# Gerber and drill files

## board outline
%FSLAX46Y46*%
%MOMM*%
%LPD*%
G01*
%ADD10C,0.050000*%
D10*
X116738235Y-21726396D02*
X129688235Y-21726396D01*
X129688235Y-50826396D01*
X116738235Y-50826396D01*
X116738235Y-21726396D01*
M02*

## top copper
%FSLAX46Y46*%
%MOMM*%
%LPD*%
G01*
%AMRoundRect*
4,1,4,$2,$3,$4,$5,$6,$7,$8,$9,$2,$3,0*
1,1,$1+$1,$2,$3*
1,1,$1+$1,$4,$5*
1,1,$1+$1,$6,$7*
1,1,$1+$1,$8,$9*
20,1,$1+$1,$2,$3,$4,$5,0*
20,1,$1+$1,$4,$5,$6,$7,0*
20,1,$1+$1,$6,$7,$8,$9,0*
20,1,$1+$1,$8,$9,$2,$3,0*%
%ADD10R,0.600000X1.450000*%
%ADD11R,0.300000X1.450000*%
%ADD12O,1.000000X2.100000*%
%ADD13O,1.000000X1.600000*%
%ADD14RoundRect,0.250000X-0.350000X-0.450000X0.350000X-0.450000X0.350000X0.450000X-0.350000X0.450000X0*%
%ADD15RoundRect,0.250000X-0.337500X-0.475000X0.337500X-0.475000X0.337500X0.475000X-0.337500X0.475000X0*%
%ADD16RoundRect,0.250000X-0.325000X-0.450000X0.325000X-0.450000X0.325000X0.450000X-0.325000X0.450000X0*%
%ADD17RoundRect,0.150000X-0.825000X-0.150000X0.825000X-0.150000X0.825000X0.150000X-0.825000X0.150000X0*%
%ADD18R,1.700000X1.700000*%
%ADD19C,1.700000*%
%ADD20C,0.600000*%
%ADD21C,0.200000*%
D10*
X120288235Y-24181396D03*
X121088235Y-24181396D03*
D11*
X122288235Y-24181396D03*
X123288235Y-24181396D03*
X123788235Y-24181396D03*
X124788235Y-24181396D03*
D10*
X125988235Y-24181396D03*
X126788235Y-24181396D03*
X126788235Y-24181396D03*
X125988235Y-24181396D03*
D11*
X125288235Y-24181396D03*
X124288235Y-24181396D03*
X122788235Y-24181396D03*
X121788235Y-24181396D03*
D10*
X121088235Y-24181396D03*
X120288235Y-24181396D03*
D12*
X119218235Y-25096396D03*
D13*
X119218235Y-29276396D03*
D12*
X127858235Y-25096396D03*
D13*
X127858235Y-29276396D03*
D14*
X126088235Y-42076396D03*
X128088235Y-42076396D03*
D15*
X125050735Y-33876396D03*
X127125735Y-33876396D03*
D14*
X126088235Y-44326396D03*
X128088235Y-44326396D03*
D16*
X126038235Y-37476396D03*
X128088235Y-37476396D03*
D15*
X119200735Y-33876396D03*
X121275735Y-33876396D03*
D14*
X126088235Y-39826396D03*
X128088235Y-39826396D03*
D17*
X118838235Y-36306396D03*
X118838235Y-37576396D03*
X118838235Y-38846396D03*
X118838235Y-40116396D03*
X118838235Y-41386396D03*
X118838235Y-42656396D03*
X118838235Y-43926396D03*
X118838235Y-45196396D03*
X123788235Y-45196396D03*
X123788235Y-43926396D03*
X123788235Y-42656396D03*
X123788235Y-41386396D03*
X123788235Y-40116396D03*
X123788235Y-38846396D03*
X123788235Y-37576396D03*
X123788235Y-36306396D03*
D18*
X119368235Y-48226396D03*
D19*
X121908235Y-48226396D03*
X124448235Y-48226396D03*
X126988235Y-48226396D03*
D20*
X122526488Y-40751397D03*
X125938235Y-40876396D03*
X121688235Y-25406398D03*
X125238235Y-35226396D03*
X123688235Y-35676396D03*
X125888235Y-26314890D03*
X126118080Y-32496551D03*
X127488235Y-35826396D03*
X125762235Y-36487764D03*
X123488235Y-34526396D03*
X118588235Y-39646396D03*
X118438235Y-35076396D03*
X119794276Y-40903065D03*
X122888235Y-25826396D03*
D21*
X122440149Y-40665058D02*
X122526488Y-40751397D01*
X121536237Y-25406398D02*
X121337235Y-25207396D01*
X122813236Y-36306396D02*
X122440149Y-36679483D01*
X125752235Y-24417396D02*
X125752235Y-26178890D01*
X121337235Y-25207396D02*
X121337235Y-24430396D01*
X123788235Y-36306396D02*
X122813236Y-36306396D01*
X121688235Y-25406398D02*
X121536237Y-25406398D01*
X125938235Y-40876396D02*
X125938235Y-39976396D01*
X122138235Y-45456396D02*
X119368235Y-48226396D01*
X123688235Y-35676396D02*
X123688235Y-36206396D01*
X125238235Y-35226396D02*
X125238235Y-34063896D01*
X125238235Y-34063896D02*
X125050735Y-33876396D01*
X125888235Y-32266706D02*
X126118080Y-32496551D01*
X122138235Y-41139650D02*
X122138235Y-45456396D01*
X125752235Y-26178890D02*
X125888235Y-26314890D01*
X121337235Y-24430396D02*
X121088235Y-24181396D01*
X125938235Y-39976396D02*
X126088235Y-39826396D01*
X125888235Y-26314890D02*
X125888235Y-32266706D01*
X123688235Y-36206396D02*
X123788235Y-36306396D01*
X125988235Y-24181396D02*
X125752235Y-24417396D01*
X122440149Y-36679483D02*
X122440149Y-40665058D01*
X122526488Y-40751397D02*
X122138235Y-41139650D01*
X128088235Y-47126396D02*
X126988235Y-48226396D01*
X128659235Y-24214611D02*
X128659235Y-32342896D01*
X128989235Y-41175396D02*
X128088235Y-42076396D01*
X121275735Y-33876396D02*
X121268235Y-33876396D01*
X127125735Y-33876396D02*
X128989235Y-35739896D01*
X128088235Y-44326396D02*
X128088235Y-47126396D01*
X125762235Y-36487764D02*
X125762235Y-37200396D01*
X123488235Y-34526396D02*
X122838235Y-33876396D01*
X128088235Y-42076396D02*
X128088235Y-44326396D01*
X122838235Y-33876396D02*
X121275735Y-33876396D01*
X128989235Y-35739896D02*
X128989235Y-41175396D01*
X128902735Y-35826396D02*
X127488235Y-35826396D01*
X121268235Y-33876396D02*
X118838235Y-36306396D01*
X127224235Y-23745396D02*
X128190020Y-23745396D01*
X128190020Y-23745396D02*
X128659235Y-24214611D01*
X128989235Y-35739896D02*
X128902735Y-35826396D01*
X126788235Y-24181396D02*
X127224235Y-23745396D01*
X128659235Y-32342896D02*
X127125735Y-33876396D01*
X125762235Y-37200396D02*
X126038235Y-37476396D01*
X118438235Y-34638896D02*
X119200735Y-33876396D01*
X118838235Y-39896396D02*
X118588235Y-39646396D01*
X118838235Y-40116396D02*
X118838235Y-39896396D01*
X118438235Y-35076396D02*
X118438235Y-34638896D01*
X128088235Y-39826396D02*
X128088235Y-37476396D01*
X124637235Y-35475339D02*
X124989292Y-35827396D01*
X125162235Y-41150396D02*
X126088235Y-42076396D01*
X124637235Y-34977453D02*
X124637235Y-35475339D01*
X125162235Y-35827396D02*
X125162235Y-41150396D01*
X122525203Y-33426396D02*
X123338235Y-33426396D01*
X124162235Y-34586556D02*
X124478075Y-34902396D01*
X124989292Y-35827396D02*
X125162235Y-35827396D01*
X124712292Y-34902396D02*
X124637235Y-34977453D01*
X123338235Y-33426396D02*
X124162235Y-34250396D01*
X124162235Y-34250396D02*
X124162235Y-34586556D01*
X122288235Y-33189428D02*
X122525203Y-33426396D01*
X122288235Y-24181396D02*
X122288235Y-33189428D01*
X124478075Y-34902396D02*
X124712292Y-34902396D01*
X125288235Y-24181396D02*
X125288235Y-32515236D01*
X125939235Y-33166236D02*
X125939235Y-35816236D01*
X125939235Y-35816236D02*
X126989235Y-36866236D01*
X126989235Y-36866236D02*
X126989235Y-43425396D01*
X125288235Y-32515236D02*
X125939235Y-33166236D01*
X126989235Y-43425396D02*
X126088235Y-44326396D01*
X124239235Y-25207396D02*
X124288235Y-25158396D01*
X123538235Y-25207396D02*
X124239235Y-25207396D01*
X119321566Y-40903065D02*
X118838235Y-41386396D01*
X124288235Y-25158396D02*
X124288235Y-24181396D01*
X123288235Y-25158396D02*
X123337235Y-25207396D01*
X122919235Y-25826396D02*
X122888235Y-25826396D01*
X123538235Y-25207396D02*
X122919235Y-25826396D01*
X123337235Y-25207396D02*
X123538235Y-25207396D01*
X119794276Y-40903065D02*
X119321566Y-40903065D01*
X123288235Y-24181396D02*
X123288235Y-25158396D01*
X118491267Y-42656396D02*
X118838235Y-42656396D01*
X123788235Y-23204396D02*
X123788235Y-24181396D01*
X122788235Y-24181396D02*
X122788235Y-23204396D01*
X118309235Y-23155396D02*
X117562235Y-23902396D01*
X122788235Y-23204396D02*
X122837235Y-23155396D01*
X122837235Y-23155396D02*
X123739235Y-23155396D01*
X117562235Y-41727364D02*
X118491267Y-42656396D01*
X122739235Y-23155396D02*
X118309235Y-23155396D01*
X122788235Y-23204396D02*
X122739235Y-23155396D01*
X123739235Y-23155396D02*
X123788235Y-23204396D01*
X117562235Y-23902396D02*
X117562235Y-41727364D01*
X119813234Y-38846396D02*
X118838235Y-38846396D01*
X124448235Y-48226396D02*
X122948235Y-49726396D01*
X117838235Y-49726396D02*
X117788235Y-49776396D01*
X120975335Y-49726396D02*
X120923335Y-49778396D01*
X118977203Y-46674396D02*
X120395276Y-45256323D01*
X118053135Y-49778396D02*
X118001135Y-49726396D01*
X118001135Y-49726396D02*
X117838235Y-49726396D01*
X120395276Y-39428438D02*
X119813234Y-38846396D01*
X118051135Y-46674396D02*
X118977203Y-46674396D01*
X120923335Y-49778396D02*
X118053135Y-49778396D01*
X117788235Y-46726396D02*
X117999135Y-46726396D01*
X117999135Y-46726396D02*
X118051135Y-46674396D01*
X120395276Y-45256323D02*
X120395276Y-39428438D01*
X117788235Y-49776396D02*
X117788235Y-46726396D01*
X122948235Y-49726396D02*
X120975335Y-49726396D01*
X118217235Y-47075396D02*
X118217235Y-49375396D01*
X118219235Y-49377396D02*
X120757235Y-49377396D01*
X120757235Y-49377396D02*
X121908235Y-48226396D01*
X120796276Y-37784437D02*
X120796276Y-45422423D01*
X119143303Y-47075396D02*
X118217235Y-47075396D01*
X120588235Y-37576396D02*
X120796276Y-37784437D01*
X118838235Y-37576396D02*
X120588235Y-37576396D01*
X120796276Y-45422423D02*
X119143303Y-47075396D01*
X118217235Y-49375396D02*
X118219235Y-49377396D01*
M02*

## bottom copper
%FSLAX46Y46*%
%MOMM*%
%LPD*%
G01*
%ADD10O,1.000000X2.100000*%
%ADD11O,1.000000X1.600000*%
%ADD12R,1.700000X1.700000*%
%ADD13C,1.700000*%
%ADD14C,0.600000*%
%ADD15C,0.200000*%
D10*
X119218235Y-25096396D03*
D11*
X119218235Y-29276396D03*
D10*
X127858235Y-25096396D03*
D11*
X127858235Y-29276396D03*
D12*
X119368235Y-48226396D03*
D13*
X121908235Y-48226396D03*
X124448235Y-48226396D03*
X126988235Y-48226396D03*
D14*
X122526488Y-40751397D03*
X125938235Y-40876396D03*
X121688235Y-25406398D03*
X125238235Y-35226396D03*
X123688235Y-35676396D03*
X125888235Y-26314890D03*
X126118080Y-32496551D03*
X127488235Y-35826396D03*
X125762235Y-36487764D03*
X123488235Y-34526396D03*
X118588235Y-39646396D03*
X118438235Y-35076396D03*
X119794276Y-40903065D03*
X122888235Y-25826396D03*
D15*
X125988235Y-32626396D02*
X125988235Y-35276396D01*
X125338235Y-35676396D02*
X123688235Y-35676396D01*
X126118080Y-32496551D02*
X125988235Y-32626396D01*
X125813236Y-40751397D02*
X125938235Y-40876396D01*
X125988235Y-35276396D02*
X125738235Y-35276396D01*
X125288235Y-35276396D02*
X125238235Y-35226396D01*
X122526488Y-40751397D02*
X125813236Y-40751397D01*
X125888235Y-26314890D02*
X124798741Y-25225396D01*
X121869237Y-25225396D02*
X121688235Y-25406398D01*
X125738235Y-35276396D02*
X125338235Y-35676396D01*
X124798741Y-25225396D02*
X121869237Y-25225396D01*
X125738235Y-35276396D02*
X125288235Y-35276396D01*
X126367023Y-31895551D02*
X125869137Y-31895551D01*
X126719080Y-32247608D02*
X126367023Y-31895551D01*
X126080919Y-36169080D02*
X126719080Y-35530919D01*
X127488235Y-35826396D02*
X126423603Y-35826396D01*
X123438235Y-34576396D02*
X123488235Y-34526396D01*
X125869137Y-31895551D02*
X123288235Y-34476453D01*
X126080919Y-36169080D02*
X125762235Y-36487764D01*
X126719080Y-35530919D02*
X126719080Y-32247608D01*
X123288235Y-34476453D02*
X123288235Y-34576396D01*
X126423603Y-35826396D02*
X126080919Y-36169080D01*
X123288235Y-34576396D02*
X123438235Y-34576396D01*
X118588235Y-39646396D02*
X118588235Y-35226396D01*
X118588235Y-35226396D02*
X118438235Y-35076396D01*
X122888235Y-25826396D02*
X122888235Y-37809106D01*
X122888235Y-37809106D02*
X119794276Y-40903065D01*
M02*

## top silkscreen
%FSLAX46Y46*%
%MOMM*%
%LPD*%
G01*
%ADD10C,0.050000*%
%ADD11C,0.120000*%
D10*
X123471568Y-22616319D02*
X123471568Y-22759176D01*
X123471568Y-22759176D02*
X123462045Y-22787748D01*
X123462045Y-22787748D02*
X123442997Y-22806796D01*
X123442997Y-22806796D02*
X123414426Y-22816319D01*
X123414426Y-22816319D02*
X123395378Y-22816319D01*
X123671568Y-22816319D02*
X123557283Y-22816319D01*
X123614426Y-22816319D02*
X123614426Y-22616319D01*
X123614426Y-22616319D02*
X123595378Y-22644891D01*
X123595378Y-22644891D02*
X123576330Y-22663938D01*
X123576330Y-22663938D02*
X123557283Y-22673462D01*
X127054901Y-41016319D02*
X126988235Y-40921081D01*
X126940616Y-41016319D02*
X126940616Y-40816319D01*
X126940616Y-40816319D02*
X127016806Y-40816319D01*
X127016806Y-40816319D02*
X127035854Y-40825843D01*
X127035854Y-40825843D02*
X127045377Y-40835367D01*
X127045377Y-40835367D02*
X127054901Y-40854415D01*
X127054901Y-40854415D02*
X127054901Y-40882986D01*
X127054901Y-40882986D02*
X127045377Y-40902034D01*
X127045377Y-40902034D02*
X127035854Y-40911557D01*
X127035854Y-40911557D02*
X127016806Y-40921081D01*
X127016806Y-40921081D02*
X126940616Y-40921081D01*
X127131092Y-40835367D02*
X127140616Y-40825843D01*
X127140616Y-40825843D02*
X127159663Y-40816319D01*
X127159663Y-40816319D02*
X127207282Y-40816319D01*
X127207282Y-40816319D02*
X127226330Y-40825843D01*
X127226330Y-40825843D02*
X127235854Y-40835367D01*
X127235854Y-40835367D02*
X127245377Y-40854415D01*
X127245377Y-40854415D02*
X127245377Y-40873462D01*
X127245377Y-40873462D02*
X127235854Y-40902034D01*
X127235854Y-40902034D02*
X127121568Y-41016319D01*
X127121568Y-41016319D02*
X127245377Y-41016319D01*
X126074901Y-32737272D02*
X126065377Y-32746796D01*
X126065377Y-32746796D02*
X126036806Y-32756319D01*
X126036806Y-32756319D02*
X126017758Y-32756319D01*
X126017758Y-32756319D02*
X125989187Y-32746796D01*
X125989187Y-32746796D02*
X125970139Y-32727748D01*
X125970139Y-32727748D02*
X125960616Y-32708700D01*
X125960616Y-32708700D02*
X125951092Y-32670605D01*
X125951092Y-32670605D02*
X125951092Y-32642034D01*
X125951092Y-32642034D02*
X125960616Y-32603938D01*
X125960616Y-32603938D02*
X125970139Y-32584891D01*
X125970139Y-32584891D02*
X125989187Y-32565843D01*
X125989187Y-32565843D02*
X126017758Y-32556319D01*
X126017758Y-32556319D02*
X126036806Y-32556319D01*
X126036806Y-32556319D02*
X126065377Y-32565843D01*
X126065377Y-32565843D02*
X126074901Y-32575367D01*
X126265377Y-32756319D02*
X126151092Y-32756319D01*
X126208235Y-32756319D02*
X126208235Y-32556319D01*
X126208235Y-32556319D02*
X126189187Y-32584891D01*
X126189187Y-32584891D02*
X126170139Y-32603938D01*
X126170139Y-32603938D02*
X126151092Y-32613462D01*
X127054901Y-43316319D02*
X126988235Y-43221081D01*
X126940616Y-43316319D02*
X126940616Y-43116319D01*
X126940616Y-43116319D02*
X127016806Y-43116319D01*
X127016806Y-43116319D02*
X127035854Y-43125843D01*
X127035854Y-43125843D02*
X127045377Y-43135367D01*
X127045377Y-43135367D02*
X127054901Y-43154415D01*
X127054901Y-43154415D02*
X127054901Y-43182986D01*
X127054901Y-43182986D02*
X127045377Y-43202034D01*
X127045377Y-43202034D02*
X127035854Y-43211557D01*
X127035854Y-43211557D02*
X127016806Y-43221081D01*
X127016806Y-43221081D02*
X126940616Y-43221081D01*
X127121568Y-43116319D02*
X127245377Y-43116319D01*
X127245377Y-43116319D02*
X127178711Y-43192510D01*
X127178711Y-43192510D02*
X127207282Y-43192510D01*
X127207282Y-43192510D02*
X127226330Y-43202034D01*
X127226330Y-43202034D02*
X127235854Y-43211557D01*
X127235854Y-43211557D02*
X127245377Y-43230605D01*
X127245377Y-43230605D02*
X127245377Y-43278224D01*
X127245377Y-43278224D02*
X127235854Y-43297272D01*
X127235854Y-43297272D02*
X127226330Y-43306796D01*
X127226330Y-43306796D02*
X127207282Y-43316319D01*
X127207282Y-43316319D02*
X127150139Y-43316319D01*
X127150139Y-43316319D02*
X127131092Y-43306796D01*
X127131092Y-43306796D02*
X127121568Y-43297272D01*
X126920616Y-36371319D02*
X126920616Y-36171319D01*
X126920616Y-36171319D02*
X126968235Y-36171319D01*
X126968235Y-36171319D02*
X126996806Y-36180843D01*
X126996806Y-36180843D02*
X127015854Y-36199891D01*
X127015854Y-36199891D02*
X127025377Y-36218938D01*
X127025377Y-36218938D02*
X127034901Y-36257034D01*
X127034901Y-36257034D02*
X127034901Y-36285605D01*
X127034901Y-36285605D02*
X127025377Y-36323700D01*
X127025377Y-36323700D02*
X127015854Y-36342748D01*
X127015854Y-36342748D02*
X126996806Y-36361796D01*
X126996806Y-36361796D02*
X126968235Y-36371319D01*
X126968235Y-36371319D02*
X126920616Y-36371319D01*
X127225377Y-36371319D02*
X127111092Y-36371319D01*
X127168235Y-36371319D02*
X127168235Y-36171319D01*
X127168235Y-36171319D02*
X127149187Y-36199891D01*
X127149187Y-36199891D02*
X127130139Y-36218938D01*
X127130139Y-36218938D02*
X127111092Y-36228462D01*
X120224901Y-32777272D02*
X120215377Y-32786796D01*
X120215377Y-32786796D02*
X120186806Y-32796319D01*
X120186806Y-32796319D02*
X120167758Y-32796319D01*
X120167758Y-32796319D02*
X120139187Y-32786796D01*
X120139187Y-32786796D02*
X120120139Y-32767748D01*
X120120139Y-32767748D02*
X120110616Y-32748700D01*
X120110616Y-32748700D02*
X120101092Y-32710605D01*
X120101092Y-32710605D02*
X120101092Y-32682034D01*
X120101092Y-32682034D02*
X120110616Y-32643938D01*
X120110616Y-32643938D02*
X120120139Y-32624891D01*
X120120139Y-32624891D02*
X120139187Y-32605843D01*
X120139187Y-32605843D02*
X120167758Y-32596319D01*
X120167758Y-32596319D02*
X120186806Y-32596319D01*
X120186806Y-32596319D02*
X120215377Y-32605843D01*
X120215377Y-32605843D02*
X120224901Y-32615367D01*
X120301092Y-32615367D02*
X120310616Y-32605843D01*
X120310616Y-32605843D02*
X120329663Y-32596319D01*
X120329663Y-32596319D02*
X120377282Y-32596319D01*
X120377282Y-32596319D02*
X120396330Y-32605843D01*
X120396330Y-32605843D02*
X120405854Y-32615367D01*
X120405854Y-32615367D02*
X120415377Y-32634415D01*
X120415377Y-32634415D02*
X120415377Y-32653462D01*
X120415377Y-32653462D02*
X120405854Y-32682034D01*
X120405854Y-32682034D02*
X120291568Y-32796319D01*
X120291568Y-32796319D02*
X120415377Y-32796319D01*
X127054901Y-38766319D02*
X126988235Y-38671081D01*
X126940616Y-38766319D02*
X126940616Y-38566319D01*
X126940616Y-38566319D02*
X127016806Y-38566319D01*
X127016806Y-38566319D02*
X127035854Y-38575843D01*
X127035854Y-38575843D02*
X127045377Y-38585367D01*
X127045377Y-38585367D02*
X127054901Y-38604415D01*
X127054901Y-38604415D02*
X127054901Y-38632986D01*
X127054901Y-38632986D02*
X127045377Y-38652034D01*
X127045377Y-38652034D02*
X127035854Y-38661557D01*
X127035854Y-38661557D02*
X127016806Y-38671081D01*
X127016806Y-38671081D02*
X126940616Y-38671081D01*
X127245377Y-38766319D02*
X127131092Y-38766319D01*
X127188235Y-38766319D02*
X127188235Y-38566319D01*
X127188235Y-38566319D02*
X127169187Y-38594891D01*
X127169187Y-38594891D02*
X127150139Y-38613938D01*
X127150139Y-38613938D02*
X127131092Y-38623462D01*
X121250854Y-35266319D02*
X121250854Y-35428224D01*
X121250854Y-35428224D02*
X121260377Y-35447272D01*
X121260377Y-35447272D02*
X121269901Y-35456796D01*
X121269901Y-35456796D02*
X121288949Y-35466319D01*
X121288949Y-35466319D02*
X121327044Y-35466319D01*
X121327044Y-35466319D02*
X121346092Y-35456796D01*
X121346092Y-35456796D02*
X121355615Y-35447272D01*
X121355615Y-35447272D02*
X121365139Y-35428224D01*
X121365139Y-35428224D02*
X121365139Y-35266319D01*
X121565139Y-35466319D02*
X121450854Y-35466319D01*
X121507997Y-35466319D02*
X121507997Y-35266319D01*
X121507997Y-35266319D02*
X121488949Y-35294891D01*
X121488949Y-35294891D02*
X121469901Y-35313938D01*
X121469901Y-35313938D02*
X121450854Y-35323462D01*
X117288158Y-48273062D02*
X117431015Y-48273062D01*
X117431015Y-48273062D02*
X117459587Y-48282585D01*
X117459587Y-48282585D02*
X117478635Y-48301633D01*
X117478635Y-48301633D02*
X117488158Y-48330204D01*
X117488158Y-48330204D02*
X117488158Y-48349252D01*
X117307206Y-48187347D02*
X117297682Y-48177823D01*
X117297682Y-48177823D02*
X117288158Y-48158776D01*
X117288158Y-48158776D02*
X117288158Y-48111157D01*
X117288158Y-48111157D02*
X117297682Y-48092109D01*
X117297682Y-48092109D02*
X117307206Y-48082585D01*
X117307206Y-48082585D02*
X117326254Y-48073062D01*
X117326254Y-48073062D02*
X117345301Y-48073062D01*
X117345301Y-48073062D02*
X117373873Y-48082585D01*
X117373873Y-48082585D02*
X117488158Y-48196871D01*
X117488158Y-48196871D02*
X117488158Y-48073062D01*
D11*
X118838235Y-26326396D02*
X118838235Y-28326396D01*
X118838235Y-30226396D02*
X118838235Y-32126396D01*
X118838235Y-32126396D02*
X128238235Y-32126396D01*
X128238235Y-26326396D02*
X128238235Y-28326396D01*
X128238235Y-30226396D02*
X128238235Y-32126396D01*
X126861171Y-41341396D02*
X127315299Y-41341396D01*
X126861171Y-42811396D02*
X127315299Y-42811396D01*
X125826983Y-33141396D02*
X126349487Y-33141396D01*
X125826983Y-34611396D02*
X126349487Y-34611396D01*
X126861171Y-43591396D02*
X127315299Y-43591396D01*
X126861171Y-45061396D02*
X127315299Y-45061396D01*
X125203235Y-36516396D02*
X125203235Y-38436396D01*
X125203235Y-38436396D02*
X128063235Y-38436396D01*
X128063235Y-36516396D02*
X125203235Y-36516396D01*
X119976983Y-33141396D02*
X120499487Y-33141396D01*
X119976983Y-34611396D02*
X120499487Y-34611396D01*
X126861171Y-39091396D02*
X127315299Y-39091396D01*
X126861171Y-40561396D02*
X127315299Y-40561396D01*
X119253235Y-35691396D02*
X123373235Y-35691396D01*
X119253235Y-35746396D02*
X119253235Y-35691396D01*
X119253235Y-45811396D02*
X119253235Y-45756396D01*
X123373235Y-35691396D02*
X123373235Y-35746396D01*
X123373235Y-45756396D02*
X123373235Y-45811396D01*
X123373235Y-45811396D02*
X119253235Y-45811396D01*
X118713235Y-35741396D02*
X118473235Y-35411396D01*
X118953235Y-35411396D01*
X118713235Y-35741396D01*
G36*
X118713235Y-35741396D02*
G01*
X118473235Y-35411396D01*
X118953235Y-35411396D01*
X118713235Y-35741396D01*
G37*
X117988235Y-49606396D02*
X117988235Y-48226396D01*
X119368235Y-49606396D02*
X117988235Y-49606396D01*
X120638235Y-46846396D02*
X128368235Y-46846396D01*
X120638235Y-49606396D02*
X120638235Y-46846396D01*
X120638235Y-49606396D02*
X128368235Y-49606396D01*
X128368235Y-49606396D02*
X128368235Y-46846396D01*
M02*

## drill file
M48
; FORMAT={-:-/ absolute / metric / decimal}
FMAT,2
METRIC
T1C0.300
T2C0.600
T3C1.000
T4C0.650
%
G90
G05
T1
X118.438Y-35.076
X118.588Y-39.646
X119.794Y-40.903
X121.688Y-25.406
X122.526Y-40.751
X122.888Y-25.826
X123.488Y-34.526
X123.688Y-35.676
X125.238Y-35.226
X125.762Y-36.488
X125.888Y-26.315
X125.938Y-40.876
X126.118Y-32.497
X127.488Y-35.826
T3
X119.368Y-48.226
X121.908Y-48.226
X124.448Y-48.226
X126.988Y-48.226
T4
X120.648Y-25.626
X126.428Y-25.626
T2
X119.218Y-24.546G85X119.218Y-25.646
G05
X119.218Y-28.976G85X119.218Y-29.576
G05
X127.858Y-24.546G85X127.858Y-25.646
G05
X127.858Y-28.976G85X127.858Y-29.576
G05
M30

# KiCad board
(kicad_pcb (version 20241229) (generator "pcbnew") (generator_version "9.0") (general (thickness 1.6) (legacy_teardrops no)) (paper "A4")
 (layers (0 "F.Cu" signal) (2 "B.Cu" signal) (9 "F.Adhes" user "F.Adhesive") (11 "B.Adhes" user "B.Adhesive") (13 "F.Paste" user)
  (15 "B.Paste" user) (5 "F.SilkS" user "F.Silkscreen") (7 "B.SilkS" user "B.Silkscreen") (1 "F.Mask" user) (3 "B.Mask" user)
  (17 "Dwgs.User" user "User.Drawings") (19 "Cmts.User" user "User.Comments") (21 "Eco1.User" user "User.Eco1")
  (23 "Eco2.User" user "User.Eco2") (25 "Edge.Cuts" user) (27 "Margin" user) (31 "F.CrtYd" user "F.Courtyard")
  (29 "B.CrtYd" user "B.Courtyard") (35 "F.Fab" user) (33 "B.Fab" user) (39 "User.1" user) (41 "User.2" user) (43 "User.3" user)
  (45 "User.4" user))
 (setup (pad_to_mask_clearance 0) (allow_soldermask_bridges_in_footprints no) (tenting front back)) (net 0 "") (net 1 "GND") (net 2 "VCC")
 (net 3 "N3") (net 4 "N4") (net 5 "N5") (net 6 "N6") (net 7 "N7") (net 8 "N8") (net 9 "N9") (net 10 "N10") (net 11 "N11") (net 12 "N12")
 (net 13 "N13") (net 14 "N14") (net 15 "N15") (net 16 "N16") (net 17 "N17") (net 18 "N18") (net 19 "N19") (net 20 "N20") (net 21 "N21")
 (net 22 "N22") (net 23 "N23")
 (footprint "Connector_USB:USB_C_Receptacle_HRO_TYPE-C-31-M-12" (layer "F.Cu") (at 123.538235 28.226396)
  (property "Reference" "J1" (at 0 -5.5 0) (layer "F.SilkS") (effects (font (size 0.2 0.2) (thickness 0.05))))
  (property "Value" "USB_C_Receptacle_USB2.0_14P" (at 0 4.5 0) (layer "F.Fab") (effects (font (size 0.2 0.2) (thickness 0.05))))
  (fp_line (start -4.7 -1.9) (end -4.7 0.1) (stroke (width 0.12) (type solid)) (layer "F.SilkS"))
  (fp_line (start -4.7 2) (end -4.7 3.9) (stroke (width 0.12) (type solid)) (layer "F.SilkS"))
  (fp_line (start -4.7 3.9) (end 4.7 3.9) (stroke (width 0.12) (type solid)) (layer "F.SilkS"))
  (fp_line (start 4.7 -1.9) (end 4.7 0.1) (stroke (width 0.12) (type solid)) (layer "F.SilkS"))
  (fp_line (start 4.7 2) (end 4.7 3.9) (stroke (width 0.12) (type solid)) (layer "F.SilkS"))
  (pad "" np_thru_hole circle (at -2.89 -2.6) (size 0.65 0.65) (drill 0.65) (layers "*.Cu" "*.Mask"))
  (pad "" np_thru_hole circle (at 2.89 -2.6) (size 0.65 0.65) (drill 0.65) (layers "*.Cu" "*.Mask"))
  (pad "A1" smd rect (at -3.25 -4.045) (size 0.6 1.45) (layers "F.Cu" "F.Mask" "F.Paste") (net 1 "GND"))
  (pad "A4" smd rect (at -2.45 -4.045) (size 0.6 1.45) (layers "F.Cu" "F.Mask" "F.Paste") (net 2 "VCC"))
  (pad "A5" smd rect (at -1.25 -4.045) (size 0.3 1.45) (layers "F.Cu" "F.Mask" "F.Paste") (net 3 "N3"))
  (pad "A6" smd rect (at -0.25 -4.045) (size 0.3 1.45) (layers "F.Cu" "F.Mask" "F.Paste") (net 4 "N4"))
  (pad "A7" smd rect (at 0.25 -4.045) (size 0.3 1.45) (layers "F.Cu" "F.Mask" "F.Paste") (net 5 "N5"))
  (pad "A8" smd rect (at 1.25 -4.045) (size 0.3 1.45) (layers "F.Cu" "F.Mask" "F.Paste"))
  (pad "A9" smd rect (at 2.45 -4.045) (size 0.6 1.45) (layers "F.Cu" "F.Mask" "F.Paste") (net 2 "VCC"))
  (pad "A12" smd rect (at 3.25 -4.045) (size 0.6 1.45) (layers "F.Cu" "F.Mask" "F.Paste") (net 1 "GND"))
  (pad "B1" smd rect (at 3.25 -4.045) (size 0.6 1.45) (layers "F.Cu" "F.Mask" "F.Paste") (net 1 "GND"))
  (pad "B4" smd rect (at 2.45 -4.045) (size 0.6 1.45) (layers "F.Cu" "F.Mask" "F.Paste") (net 2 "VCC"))
  (pad "B5" smd rect (at 1.75 -4.045) (size 0.3 1.45) (layers "F.Cu" "F.Mask" "F.Paste") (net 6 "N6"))
  (pad "B6" smd rect (at 0.75 -4.045) (size 0.3 1.45) (layers "F.Cu" "F.Mask" "F.Paste") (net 4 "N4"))
  (pad "B7" smd rect (at -0.75 -4.045) (size 0.3 1.45) (layers "F.Cu" "F.Mask" "F.Paste") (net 5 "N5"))
  (pad "B8" smd rect (at -1.75 -4.045) (size 0.3 1.45) (layers "F.Cu" "F.Mask" "F.Paste"))
  (pad "B9" smd rect (at -2.45 -4.045) (size 0.6 1.45) (layers "F.Cu" "F.Mask" "F.Paste") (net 2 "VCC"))
  (pad "B12" smd rect (at -3.25 -4.045) (size 0.6 1.45) (layers "F.Cu" "F.Mask" "F.Paste") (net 1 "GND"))
  (pad "S1" thru_hole oval (at -4.32 -3.13) (size 1 2.1) (drill oval 0.6 1.7) (layers "*.Cu" "*.Mask") (remove_unused_layers no)
   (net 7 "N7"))
  (pad "S1" thru_hole oval (at -4.32 1.05) (size 1 1.6) (drill oval 0.6 1.2) (layers "*.Cu" "*.Mask") (remove_unused_layers no) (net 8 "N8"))
  (pad "S1" thru_hole oval (at 4.32 -3.13) (size 1 2.1) (drill oval 0.6 1.7) (layers "*.Cu" "*.Mask") (remove_unused_layers no) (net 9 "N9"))
  (pad "S1" thru_hole oval (at 4.32 1.05) (size 1 1.6) (drill oval 0.6 1.2) (layers "*.Cu" "*.Mask") (remove_unused_layers no)
   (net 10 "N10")))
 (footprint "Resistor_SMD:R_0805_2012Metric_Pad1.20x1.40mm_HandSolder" (layer "F.Cu") (at 127.088235 42.076396)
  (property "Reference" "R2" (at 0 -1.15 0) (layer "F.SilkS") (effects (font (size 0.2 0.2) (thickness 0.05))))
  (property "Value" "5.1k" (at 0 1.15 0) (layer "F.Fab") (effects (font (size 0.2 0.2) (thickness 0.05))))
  (fp_line (start -0.227064 -0.735) (end 0.227064 -0.735) (stroke (width 0.12) (type solid)) (layer "F.SilkS"))
  (fp_line (start -0.227064 0.735) (end 0.227064 0.735) (stroke (width 0.12) (type solid)) (layer "F.SilkS"))
  (pad "1" smd roundrect (at -1 0) (size 1.2 1.4) (layers "F.Cu" "F.Mask" "F.Paste") (roundrect_rratio 0.208333) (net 3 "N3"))
  (pad "2" smd roundrect (at 1 0) (size 1.2 1.4) (layers "F.Cu" "F.Mask" "F.Paste") (roundrect_rratio 0.208333) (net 1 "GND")))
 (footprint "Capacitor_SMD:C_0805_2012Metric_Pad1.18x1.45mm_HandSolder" (layer "F.Cu") (at 126.088235 33.876396)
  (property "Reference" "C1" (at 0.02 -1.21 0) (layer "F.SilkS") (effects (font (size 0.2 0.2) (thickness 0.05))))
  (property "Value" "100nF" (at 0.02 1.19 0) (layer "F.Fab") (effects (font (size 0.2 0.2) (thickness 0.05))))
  (fp_line (start -0.261252 -0.735) (end 0.261252 -0.735) (stroke (width 0.12) (type solid)) (layer "F.SilkS"))
  (fp_line (start -0.261252 0.735) (end 0.261252 0.735) (stroke (width 0.12) (type solid)) (layer "F.SilkS"))
  (pad "1" smd roundrect (at -1.0375 0) (size 1.175 1.45) (layers "F.Cu" "F.Mask" "F.Paste") (roundrect_rratio 0.212766) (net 2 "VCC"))
  (pad "2" smd roundrect (at 1.0375 0) (size 1.175 1.45) (layers "F.Cu" "F.Mask" "F.Paste") (roundrect_rratio 0.212766) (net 1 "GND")))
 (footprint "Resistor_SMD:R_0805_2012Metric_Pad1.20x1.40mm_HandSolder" (layer "F.Cu") (at 127.088235 44.326396)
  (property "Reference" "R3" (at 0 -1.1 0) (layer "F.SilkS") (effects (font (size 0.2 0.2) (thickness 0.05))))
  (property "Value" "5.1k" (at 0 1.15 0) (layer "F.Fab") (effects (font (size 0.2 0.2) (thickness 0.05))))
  (fp_line (start -0.227064 -0.735) (end 0.227064 -0.735) (stroke (width 0.12) (type solid)) (layer "F.SilkS"))
  (fp_line (start -0.227064 0.735) (end 0.227064 0.735) (stroke (width 0.12) (type solid)) (layer "F.SilkS"))
  (pad "1" smd roundrect (at -1 0) (size 1.2 1.4) (layers "F.Cu" "F.Mask" "F.Paste") (roundrect_rratio 0.208333) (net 6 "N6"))
  (pad "2" smd roundrect (at 1 0) (size 1.2 1.4) (layers "F.Cu" "F.Mask" "F.Paste") (roundrect_rratio 0.208333) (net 1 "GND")))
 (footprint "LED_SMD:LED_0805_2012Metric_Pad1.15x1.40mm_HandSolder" (layer "F.Cu") (at 127.063235 37.476396)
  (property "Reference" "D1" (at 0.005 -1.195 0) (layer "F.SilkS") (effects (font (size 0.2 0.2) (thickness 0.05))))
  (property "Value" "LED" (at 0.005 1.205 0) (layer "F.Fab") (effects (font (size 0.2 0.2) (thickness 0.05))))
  (fp_line (start -1.86 -0.96) (end -1.86 0.96) (stroke (width 0.12) (type solid)) (layer "F.SilkS"))
  (fp_line (start -1.86 0.96) (end 1 0.96) (stroke (width 0.12) (type solid)) (layer "F.SilkS"))
  (fp_line (start 1 -0.96) (end -1.86 -0.96) (stroke (width 0.12) (type solid)) (layer "F.SilkS"))
  (pad "1" smd roundrect (at -1.025 0) (size 1.15 1.4) (layers "F.Cu" "F.Mask" "F.Paste") (roundrect_rratio 0.217391) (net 1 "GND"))
  (pad "2" smd roundrect (at 1.025 0) (size 1.15 1.4) (layers "F.Cu" "F.Mask" "F.Paste") (roundrect_rratio 0.217391) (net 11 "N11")))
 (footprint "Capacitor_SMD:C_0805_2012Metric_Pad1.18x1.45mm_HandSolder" (layer "F.Cu") (at 120.238235 33.876396)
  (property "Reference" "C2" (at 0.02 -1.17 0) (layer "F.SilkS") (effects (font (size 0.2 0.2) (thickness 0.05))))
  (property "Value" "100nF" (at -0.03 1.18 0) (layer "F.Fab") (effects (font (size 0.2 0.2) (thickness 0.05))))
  (fp_line (start -0.261252 -0.735) (end 0.261252 -0.735) (stroke (width 0.12) (type solid)) (layer "F.SilkS"))
  (fp_line (start -0.261252 0.735) (end 0.261252 0.735) (stroke (width 0.12) (type solid)) (layer "F.SilkS"))
  (pad "1" smd roundrect (at -1.0375 0) (size 1.175 1.45) (layers "F.Cu" "F.Mask" "F.Paste") (roundrect_rratio 0.212766) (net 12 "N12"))
  (pad "2" smd roundrect (at 1.0375 0) (size 1.175 1.45) (layers "F.Cu" "F.Mask" "F.Paste") (roundrect_rratio 0.212766) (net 1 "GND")))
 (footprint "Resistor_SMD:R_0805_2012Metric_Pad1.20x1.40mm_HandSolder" (layer "F.Cu") (at 127.088235 39.826396)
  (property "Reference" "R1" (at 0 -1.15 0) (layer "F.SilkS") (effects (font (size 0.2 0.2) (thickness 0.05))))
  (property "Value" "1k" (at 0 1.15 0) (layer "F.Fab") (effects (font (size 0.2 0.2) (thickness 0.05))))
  (fp_line (start -0.227064 -0.735) (end 0.227064 -0.735) (stroke (width 0.12) (type solid)) (layer "F.SilkS"))
  (fp_line (start -0.227064 0.735) (end 0.227064 0.735) (stroke (width 0.12) (type solid)) (layer "F.SilkS"))
  (pad "1" smd roundrect (at -1 0) (size 1.2 1.4) (layers "F.Cu" "F.Mask" "F.Paste") (roundrect_rratio 0.208333) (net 2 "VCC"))
  (pad "2" smd roundrect (at 1 0) (size 1.2 1.4) (layers "F.Cu" "F.Mask" "F.Paste") (roundrect_rratio 0.208333) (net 11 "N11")))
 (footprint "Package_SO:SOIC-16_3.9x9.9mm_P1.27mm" (layer "F.Cu") (at 121.313235 40.751396)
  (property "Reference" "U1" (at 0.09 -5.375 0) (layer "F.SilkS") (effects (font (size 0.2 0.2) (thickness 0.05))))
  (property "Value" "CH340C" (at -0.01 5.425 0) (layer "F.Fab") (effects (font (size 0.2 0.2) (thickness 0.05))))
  (fp_line (start -2.06 -5.06) (end 2.06 -5.06) (stroke (width 0.12) (type solid)) (layer "F.SilkS"))
  (fp_line (start -2.06 -5.005) (end -2.06 -5.06) (stroke (width 0.12) (type solid)) (layer "F.SilkS"))
  (fp_line (start -2.06 5.06) (end -2.06 5.005) (stroke (width 0.12) (type solid)) (layer "F.SilkS"))
  (fp_line (start 2.06 -5.06) (end 2.06 -5.005) (stroke (width 0.12) (type solid)) (layer "F.SilkS"))
  (fp_line (start 2.06 5.005) (end 2.06 5.06) (stroke (width 0.12) (type solid)) (layer "F.SilkS"))
  (fp_line (start 2.06 5.06) (end -2.06 5.06) (stroke (width 0.12) (type solid)) (layer "F.SilkS"))
  (fp_poly (pts (xy -2.6 -5.01) (xy -2.84 -5.34) (xy -2.36 -5.34)) (stroke (width 0.12) (type solid)) (fill yes) (layer "F.SilkS"))
  (pad "1" smd roundrect (at -2.475 -4.445) (size 1.95 0.6) (layers "F.Cu" "F.Mask" "F.Paste") (roundrect_rratio 0.25) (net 1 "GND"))
  (pad "2" smd roundrect (at -2.475 -3.175) (size 1.95 0.6) (layers "F.Cu" "F.Mask" "F.Paste") (roundrect_rratio 0.25) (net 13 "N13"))
  (pad "3" smd roundrect (at -2.475 -1.905) (size 1.95 0.6) (layers "F.Cu" "F.Mask" "F.Paste") (roundrect_rratio 0.25) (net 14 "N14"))
  (pad "4" smd roundrect (at -2.475 -0.635) (size 1.95 0.6) (layers "F.Cu" "F.Mask" "F.Paste") (roundrect_rratio 0.25) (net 12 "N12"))
  (pad "5" smd roundrect (at -2.475 0.635) (size 1.95 0.6) (layers "F.Cu" "F.Mask" "F.Paste") (roundrect_rratio 0.25) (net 4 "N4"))
  (pad "6" smd roundrect (at -2.475 1.905) (size 1.95 0.6) (layers "F.Cu" "F.Mask" "F.Paste") (roundrect_rratio 0.25) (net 5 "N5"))
  (pad "7" smd roundrect (at -2.475 3.175) (size 1.95 0.6) (layers "F.Cu" "F.Mask" "F.Paste") (roundrect_rratio 0.25) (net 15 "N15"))
  (pad "8" smd roundrect (at -2.475 4.445) (size 1.95 0.6) (layers "F.Cu" "F.Mask" "F.Paste") (roundrect_rratio 0.25) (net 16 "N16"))
  (pad "9" smd roundrect (at 2.475 4.445) (size 1.95 0.6) (layers "F.Cu" "F.Mask" "F.Paste") (roundrect_rratio 0.25) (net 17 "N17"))
  (pad "10" smd roundrect (at 2.475 3.175) (size 1.95 0.6) (layers "F.Cu" "F.Mask" "F.Paste") (roundrect_rratio 0.25) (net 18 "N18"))
  (pad "11" smd roundrect (at 2.475 1.905) (size 1.95 0.6) (layers "F.Cu" "F.Mask" "F.Paste") (roundrect_rratio 0.25) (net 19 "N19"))
  (pad "12" smd roundrect (at 2.475 0.635) (size 1.95 0.6) (layers "F.Cu" "F.Mask" "F.Paste") (roundrect_rratio 0.25) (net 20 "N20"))
  (pad "13" smd roundrect (at 2.475 -0.635) (size 1.95 0.6) (layers "F.Cu" "F.Mask" "F.Paste") (roundrect_rratio 0.25) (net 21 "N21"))
  (pad "14" smd roundrect (at 2.475 -1.905) (size 1.95 0.6) (layers "F.Cu" "F.Mask" "F.Paste") (roundrect_rratio 0.25) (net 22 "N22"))
  (pad "15" smd roundrect (at 2.475 -3.175) (size 1.95 0.6) (layers "F.Cu" "F.Mask" "F.Paste") (roundrect_rratio 0.25) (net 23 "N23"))
  (pad "16" smd roundrect (at 2.475 -4.445) (size 1.95 0.6) (layers "F.Cu" "F.Mask" "F.Paste") (roundrect_rratio 0.25) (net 2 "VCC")))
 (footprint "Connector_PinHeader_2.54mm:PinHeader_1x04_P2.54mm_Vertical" (layer "F.Cu") (at 119.368235 48.226396 90)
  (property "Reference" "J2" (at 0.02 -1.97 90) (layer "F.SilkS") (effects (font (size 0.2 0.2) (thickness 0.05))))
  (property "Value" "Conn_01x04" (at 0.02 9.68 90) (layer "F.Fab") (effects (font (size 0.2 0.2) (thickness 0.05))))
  (fp_line (start -1.38 -1.38) (end 0 -1.38) (stroke (width 0.12) (type solid)) (layer "F.SilkS"))
  (fp_line (start -1.38 0) (end -1.38 -1.38) (stroke (width 0.12) (type solid)) (layer "F.SilkS"))
  (fp_line (start 1.38 1.27) (end 1.38 9) (stroke (width 0.12) (type solid)) (layer "F.SilkS"))
  (fp_line (start -1.38 1.27) (end 1.38 1.27) (stroke (width 0.12) (type solid)) (layer "F.SilkS"))
  (fp_line (start -1.38 1.27) (end -1.38 9) (stroke (width 0.12) (type solid)) (layer "F.SilkS"))
  (fp_line (start -1.38 9) (end 1.38 9) (stroke (width 0.12) (type solid)) (layer "F.SilkS"))
  (pad "1" thru_hole rect (at 0 0 90) (size 1.7 1.7) (drill 1) (layers "*.Cu" "*.Mask") (remove_unused_layers no) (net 2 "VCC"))
  (pad "2" thru_hole circle (at 0 2.54 90) (size 1.7 1.7) (drill 1) (layers "*.Cu" "*.Mask") (remove_unused_layers no) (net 13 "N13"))
  (pad "3" thru_hole circle (at 0 5.08 90) (size 1.7 1.7) (drill 1) (layers "*.Cu" "*.Mask") (remove_unused_layers no) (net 14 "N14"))
  (pad "4" thru_hole circle (at 0 7.62 90) (size 1.7 1.7) (drill 1) (layers "*.Cu" "*.Mask") (remove_unused_layers no) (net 1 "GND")))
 (gr_rect (start 116.738235 21.726396) (end 129.688235 50.826396) (stroke (width 0.05) (type default)) (fill no) (layer "Edge.Cuts"))
 (segment (start 122.440149 40.665058) (end 122.526488 40.751397) (width 0.2) (layer "F.Cu") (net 2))
 (segment (start 121.536237 25.406398) (end 121.337235 25.207396) (width 0.2) (layer "F.Cu") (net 2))
 (segment (start 122.813236 36.306396) (end 122.440149 36.679483) (width 0.2) (layer "F.Cu") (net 2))
 (segment (start 125.752235 24.417396) (end 125.752235 26.17889) (width 0.2) (layer "F.Cu") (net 2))
 (segment (start 121.337235 25.207396) (end 121.337235 24.430396) (width 0.2) (layer "F.Cu") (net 2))
 (segment (start 123.788235 36.306396) (end 122.813236 36.306396) (width 0.2) (layer "F.Cu") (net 2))
 (segment (start 121.688235 25.406398) (end 121.536237 25.406398) (width 0.2) (layer "F.Cu") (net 2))
 (segment (start 125.938235 40.876396) (end 125.938235 39.976396) (width 0.2) (layer "F.Cu") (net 2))
 (segment (start 122.138235 45.456396) (end 119.368235 48.226396) (width 0.2) (layer "F.Cu") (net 2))
 (segment (start 123.688235 35.676396) (end 123.688235 36.206396) (width 0.2) (layer "F.Cu") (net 2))
 (segment (start 125.238235 35.226396) (end 125.238235 34.063896) (width 0.2) (layer "F.Cu") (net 2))
 (segment (start 125.238235 34.063896) (end 125.050735 33.876396) (width 0.2) (layer "F.Cu") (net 2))
 (segment (start 125.888235 32.266706) (end 126.11808 32.496551) (width 0.2) (layer "F.Cu") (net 2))
 (segment (start 122.138235 41.13965) (end 122.138235 45.456396) (width 0.2) (layer "F.Cu") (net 2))
 (segment (start 125.752235 26.17889) (end 125.888235 26.31489) (width 0.2) (layer "F.Cu") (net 2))
 (segment (start 121.337235 24.430396) (end 121.088235 24.181396) (width 0.2) (layer "F.Cu") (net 2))
 (segment (start 125.938235 39.976396) (end 126.088235 39.826396) (width 0.2) (layer "F.Cu") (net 2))
 (segment (start 125.888235 26.31489) (end 125.888235 32.266706) (width 0.2) (layer "F.Cu") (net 2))
 (segment (start 123.688235 36.206396) (end 123.788235 36.306396) (width 0.2) (layer "F.Cu") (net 2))
 (segment (start 125.988235 24.181396) (end 125.752235 24.417396) (width 0.2) (layer "F.Cu") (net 2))
 (segment (start 122.440149 36.679483) (end 122.440149 40.665058) (width 0.2) (layer "F.Cu") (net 2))
 (segment (start 122.526488 40.751397) (end 122.138235 41.13965) (width 0.2) (layer "F.Cu") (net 2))
 (via (at 122.526488 40.751397) (size 0.6) (drill 0.3) (layers "F.Cu" "B.Cu") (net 2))
 (via (at 125.938235 40.876396) (size 0.6) (drill 0.3) (layers "F.Cu" "B.Cu") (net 2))
 (via (at 121.688235 25.406398) (size 0.6) (drill 0.3) (layers "F.Cu" "B.Cu") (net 2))
 (via (at 125.238235 35.226396) (size 0.6) (drill 0.3) (layers "F.Cu" "B.Cu") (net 2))
 (via (at 123.688235 35.676396) (size 0.6) (drill 0.3) (layers "F.Cu" "B.Cu") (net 2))
 (via (at 125.888235 26.31489) (size 0.6) (drill 0.3) (layers "F.Cu" "B.Cu") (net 2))
 (via (at 126.11808 32.496551) (size 0.6) (drill 0.3) (layers "F.Cu" "B.Cu") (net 2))
 (segment (start 125.988235 32.626396) (end 125.988235 35.276396) (width 0.2) (layer "B.Cu") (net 2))
 (segment (start 125.338235 35.676396) (end 123.688235 35.676396) (width 0.2) (layer "B.Cu") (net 2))
 (segment (start 126.11808 32.496551) (end 125.988235 32.626396) (width 0.2) (layer "B.Cu") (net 2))
 (segment (start 125.813236 40.751397) (end 125.938235 40.876396) (width 0.2) (layer "B.Cu") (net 2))
 (segment (start 125.988235 35.276396) (end 125.738235 35.276396) (width 0.2) (layer "B.Cu") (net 2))
 (segment (start 125.288235 35.276396) (end 125.238235 35.226396) (width 0.2) (layer "B.Cu") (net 2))
 (segment (start 122.526488 40.751397) (end 125.813236 40.751397) (width 0.2) (layer "B.Cu") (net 2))
 (segment (start 125.888235 26.31489) (end 124.798741 25.225396) (width 0.2) (layer "B.Cu") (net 2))
 (segment (start 121.869237 25.225396) (end 121.688235 25.406398) (width 0.2) (layer "B.Cu") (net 2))
 (segment (start 125.738235 35.276396) (end 125.338235 35.676396) (width 0.2) (layer "B.Cu") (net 2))
 (segment (start 124.798741 25.225396) (end 121.869237 25.225396) (width 0.2) (layer "B.Cu") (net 2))
 (segment (start 125.738235 35.276396) (end 125.288235 35.276396) (width 0.2) (layer "B.Cu") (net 2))
 (segment (start 128.088235 47.126396) (end 126.988235 48.226396) (width 0.2) (layer "F.Cu") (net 1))
 (segment (start 128.659235 24.214611) (end 128.659235 32.342896) (width 0.2) (layer "F.Cu") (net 1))
 (segment (start 128.989235 41.175396) (end 128.088235 42.076396) (width 0.2) (layer "F.Cu") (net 1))
 (segment (start 121.275735 33.876396) (end 121.268235 33.876396) (width 0.2) (layer "F.Cu") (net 1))
 (segment (start 127.125735 33.876396) (end 128.989235 35.739896) (width 0.2) (layer "F.Cu") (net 1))
 (segment (start 128.088235 44.326396) (end 128.088235 47.126396) (width 0.2) (layer "F.Cu") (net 1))
 (segment (start 125.762235 36.487764) (end 125.762235 37.200396) (width 0.2) (layer "F.Cu") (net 1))
 (segment (start 123.488235 34.526396) (end 122.838235 33.876396) (width 0.2) (layer "F.Cu") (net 1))
 (segment (start 128.088235 42.076396) (end 128.088235 44.326396) (width 0.2) (layer "F.Cu") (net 1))
 (segment (start 122.838235 33.876396) (end 121.275735 33.876396) (width 0.2) (layer "F.Cu") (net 1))
 (segment (start 128.989235 35.739896) (end 128.989235 41.175396) (width 0.2) (layer "F.Cu") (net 1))
 (segment (start 128.902735 35.826396) (end 127.488235 35.826396) (width 0.2) (layer "F.Cu") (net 1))
 (segment (start 121.268235 33.876396) (end 118.838235 36.306396) (width 0.2) (layer "F.Cu") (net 1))
 (segment (start 127.224235 23.745396) (end 128.19002 23.745396) (width 0.2) (layer "F.Cu") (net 1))
 (segment (start 128.19002 23.745396) (end 128.659235 24.214611) (width 0.2) (layer "F.Cu") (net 1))
 (segment (start 128.989235 35.739896) (end 128.902735 35.826396) (width 0.2) (layer "F.Cu") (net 1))
 (segment (start 126.788235 24.181396) (end 127.224235 23.745396) (width 0.2) (layer "F.Cu") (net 1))
 (segment (start 128.659235 32.342896) (end 127.125735 33.876396) (width 0.2) (layer "F.Cu") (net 1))
 (segment (start 125.762235 37.200396) (end 126.038235 37.476396) (width 0.2) (layer "F.Cu") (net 1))
 (via (at 127.488235 35.826396) (size 0.6) (drill 0.3) (layers "F.Cu" "B.Cu") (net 1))
 (via (at 125.762235 36.487764) (size 0.6) (drill 0.3) (layers "F.Cu" "B.Cu") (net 1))
 (via (at 123.488235 34.526396) (size 0.6) (drill 0.3) (layers "F.Cu" "B.Cu") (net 1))
 (segment (start 126.367023 31.895551) (end 125.869137 31.895551) (width 0.2) (layer "B.Cu") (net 1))
 (segment (start 126.71908 32.247608) (end 126.367023 31.895551) (width 0.2) (layer "B.Cu") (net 1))
 (segment (start 126.080919 36.16908) (end 126.71908 35.530919) (width 0.2) (layer "B.Cu") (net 1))
 (segment (start 127.488235 35.826396) (end 126.423603 35.826396) (width 0.2) (layer "B.Cu") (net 1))
 (segment (start 123.438235 34.576396) (end 123.488235 34.526396) (width 0.2) (layer "B.Cu") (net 1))
 (segment (start 125.869137 31.895551) (end 123.288235 34.476453) (width 0.2) (layer "B.Cu") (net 1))
 (segment (start 126.080919 36.16908) (end 125.762235 36.487764) (width 0.2) (layer "B.Cu") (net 1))
 (segment (start 126.71908 35.530919) (end 126.71908 32.247608) (width 0.2) (layer "B.Cu") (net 1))
 (segment (start 123.288235 34.476453) (end 123.288235 34.576396) (width 0.2) (layer "B.Cu") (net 1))
 (segment (start 126.423603 35.826396) (end 126.080919 36.16908) (width 0.2) (layer "B.Cu") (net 1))
 (segment (start 123.288235 34.576396) (end 123.438235 34.576396) (width 0.2) (layer "B.Cu") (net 1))
 (segment (start 118.438235 34.638896) (end 119.200735 33.876396) (width 0.2) (layer "F.Cu") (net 12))
 (segment (start 118.838235 39.896396) (end 118.588235 39.646396) (width 0.2) (layer "F.Cu") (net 12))
 (segment (start 118.838235 40.116396) (end 118.838235 39.896396) (width 0.2) (layer "F.Cu") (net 12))
 (segment (start 118.438235 35.076396) (end 118.438235 34.638896) (width 0.2) (layer "F.Cu") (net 12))
 (via (at 118.588235 39.646396) (size 0.6) (drill 0.3) (layers "F.Cu" "B.Cu") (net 12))
 (via (at 118.438235 35.076396) (size 0.6) (drill 0.3) (layers "F.Cu" "B.Cu") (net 12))
 (segment (start 118.588235 39.646396) (end 118.588235 35.226396) (width 0.2) (layer "B.Cu") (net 12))
 (segment (start 118.588235 35.226396) (end 118.438235 35.076396) (width 0.2) (layer "B.Cu") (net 12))
 (segment (start 128.088235 39.826396) (end 128.088235 37.476396) (width 0.2) (layer "F.Cu") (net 11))
 (segment (start 124.637235 35.475339) (end 124.989292 35.827396) (width 0.2) (layer "F.Cu") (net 3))
 (segment (start 125.162235 41.150396) (end 126.088235 42.076396) (width 0.2) (layer "F.Cu") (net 3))
 (segment (start 124.637235 34.977453) (end 124.637235 35.475339) (width 0.2) (layer "F.Cu") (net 3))
 (segment (start 125.162235 35.827396) (end 125.162235 41.150396) (width 0.2) (layer "F.Cu") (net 3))
 (segment (start 122.525203 33.426396) (end 123.338235 33.426396) (width 0.2) (layer "F.Cu") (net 3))
 (segment (start 124.162235 34.586556) (end 124.478075 34.902396) (width 0.2) (layer "F.Cu") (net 3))
 (segment (start 124.989292 35.827396) (end 125.162235 35.827396) (width 0.2) (layer "F.Cu") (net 3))
 (segment (start 124.712292 34.902396) (end 124.637235 34.977453) (width 0.2) (layer "F.Cu") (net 3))
 (segment (start 123.338235 33.426396) (end 124.162235 34.250396) (width 0.2) (layer "F.Cu") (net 3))
 (segment (start 124.162235 34.250396) (end 124.162235 34.586556) (width 0.2) (layer "F.Cu") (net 3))
 (segment (start 122.288235 33.189428) (end 122.525203 33.426396) (width 0.2) (layer "F.Cu") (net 3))
 (segment (start 122.288235 24.181396) (end 122.288235 33.189428) (width 0.2) (layer "F.Cu") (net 3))
 (segment (start 124.478075 34.902396) (end 124.712292 34.902396) (width 0.2) (layer "F.Cu") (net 3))
 (segment (start 125.288235 24.181396) (end 125.288235 32.515236) (width 0.2) (layer "F.Cu") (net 6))
 (segment (start 125.939235 33.166236) (end 125.939235 35.816236) (width 0.2) (layer "F.Cu") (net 6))
 (segment (start 125.939235 35.816236) (end 126.989235 36.866236) (width 0.2) (layer "F.Cu") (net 6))
 (segment (start 126.989235 36.866236) (end 126.989235 43.425396) (width 0.2) (layer "F.Cu") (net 6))
 (segment (start 125.288235 32.515236) (end 125.939235 33.166236) (width 0.2) (layer "F.Cu") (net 6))
 (segment (start 126.989235 43.425396) (end 126.088235 44.326396) (width 0.2) (layer "F.Cu") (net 6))
 (segment (start 124.239235 25.207396) (end 124.288235 25.158396) (width 0.2) (layer "F.Cu") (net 4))
 (segment (start 123.538235 25.207396) (end 124.239235 25.207396) (width 0.2) (layer "F.Cu") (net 4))
 (segment (start 119.321566 40.903065) (end 118.838235 41.386396) (width 0.2) (layer "F.Cu") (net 4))
 (segment (start 124.288235 25.158396) (end 124.288235 24.181396) (width 0.2) (layer "F.Cu") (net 4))
 (segment (start 123.288235 25.158396) (end 123.337235 25.207396) (width 0.2) (layer "F.Cu") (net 4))
 (segment (start 122.919235 25.826396) (end 122.888235 25.826396) (width 0.2) (layer "F.Cu") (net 4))
 (segment (start 123.538235 25.207396) (end 122.919235 25.826396) (width 0.2) (layer "F.Cu") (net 4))
 (segment (start 123.337235 25.207396) (end 123.538235 25.207396) (width 0.2) (layer "F.Cu") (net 4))
 (segment (start 119.794276 40.903065) (end 119.321566 40.903065) (width 0.2) (layer "F.Cu") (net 4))
 (segment (start 123.288235 24.181396) (end 123.288235 25.158396) (width 0.2) (layer "F.Cu") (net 4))
 (via (at 119.794276 40.903065) (size 0.6) (drill 0.3) (layers "F.Cu" "B.Cu") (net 4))
 (via (at 122.888235 25.826396) (size 0.6) (drill 0.3) (layers "F.Cu" "B.Cu") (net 4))
 (segment (start 122.888235 25.826396) (end 122.888235 37.809106) (width 0.2) (layer "B.Cu") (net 4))
 (segment (start 122.888235 37.809106) (end 119.794276 40.903065) (width 0.2) (layer "B.Cu") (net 4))
 (segment (start 118.491267 42.656396) (end 118.838235 42.656396) (width 0.2) (layer "F.Cu") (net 5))
 (segment (start 123.788235 23.204396) (end 123.788235 24.181396) (width 0.2) (layer "F.Cu") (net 5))
 (segment (start 122.788235 24.181396) (end 122.788235 23.204396) (width 0.2) (layer "F.Cu") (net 5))
 (segment (start 118.309235 23.155396) (end 117.562235 23.902396) (width 0.2) (layer "F.Cu") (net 5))
 (segment (start 122.788235 23.204396) (end 122.837235 23.155396) (width 0.2) (layer "F.Cu") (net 5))
 (segment (start 122.837235 23.155396) (end 123.739235 23.155396) (width 0.2) (layer "F.Cu") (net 5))
 (segment (start 117.562235 41.727364) (end 118.491267 42.656396) (width 0.2) (layer "F.Cu") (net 5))
 (segment (start 122.739235 23.155396) (end 118.309235 23.155396) (width 0.2) (layer "F.Cu") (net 5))
 (segment (start 122.788235 23.204396) (end 122.739235 23.155396) (width 0.2) (layer "F.Cu") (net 5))
 (segment (start 123.739235 23.155396) (end 123.788235 23.204396) (width 0.2) (layer "F.Cu") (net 5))
 (segment (start 117.562235 23.902396) (end 117.562235 41.727364) (width 0.2) (layer "F.Cu") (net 5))
 (segment (start 119.813234 38.846396) (end 118.838235 38.846396) (width 0.2) (layer "F.Cu") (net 14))
 (segment (start 124.448235 48.226396) (end 122.948235 49.726396) (width 0.2) (layer "F.Cu") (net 14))
 (segment (start 117.838235 49.726396) (end 117.788235 49.776396) (width 0.2) (layer "F.Cu") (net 14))
 (segment (start 120.975335 49.726396) (end 120.923335 49.778396) (width 0.2) (layer "F.Cu") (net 14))
 (segment (start 118.977203 46.674396) (end 120.395276 45.256323) (width 0.2) (layer "F.Cu") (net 14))
 (segment (start 118.053135 49.778396) (end 118.001135 49.726396) (width 0.2) (layer "F.Cu") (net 14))
 (segment (start 118.001135 49.726396) (end 117.838235 49.726396) (width 0.2) (layer "F.Cu") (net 14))
 (segment (start 120.395276 39.428438) (end 119.813234 38.846396) (width 0.2) (layer "F.Cu") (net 14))
 (segment (start 118.051135 46.674396) (end 118.977203 46.674396) (width 0.2) (layer "F.Cu") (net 14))
 (segment (start 120.923335 49.778396) (end 118.053135 49.778396) (width 0.2) (layer "F.Cu") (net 14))
 (segment (start 117.788235 46.726396) (end 117.999135 46.726396) (width 0.2) (layer "F.Cu") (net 14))
 (segment (start 117.999135 46.726396) (end 118.051135 46.674396) (width 0.2) (layer "F.Cu") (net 14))
 (segment (start 120.395276 45.256323) (end 120.395276 39.428438) (width 0.2) (layer "F.Cu") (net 14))
 (segment (start 117.788235 49.776396) (end 117.788235 46.726396) (width 0.2) (layer "F.Cu") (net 14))
 (segment (start 122.948235 49.726396) (end 120.975335 49.726396) (width 0.2) (layer "F.Cu") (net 14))
 (segment (start 118.217235 47.075396) (end 118.217235 49.375396) (width 0.2) (layer "F.Cu") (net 13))
 (segment (start 118.219235 49.377396) (end 120.757235 49.377396) (width 0.2) (layer "F.Cu") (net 13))
 (segment (start 120.757235 49.377396) (end 121.908235 48.226396) (width 0.2) (layer "F.Cu") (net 13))
 (segment (start 120.796276 37.784437) (end 120.796276 45.422423) (width 0.2) (layer "F.Cu") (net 13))
 (segment (start 119.143303 47.075396) (end 118.217235 47.075396) (width 0.2) (layer "F.Cu") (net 13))
 (segment (start 120.588235 37.576396) (end 120.796276 37.784437) (width 0.2) (layer "F.Cu") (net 13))
 (segment (start 118.838235 37.576396) (end 120.588235 37.576396) (width 0.2) (layer "F.Cu") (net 13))
 (segment (start 120.796276 45.422423) (end 119.143303 47.075396) (width 0.2) (layer "F.Cu") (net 13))
 (segment (start 118.217235 49.375396) (end 118.219235 49.377396) (width 0.2) (layer "F.Cu") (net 13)))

